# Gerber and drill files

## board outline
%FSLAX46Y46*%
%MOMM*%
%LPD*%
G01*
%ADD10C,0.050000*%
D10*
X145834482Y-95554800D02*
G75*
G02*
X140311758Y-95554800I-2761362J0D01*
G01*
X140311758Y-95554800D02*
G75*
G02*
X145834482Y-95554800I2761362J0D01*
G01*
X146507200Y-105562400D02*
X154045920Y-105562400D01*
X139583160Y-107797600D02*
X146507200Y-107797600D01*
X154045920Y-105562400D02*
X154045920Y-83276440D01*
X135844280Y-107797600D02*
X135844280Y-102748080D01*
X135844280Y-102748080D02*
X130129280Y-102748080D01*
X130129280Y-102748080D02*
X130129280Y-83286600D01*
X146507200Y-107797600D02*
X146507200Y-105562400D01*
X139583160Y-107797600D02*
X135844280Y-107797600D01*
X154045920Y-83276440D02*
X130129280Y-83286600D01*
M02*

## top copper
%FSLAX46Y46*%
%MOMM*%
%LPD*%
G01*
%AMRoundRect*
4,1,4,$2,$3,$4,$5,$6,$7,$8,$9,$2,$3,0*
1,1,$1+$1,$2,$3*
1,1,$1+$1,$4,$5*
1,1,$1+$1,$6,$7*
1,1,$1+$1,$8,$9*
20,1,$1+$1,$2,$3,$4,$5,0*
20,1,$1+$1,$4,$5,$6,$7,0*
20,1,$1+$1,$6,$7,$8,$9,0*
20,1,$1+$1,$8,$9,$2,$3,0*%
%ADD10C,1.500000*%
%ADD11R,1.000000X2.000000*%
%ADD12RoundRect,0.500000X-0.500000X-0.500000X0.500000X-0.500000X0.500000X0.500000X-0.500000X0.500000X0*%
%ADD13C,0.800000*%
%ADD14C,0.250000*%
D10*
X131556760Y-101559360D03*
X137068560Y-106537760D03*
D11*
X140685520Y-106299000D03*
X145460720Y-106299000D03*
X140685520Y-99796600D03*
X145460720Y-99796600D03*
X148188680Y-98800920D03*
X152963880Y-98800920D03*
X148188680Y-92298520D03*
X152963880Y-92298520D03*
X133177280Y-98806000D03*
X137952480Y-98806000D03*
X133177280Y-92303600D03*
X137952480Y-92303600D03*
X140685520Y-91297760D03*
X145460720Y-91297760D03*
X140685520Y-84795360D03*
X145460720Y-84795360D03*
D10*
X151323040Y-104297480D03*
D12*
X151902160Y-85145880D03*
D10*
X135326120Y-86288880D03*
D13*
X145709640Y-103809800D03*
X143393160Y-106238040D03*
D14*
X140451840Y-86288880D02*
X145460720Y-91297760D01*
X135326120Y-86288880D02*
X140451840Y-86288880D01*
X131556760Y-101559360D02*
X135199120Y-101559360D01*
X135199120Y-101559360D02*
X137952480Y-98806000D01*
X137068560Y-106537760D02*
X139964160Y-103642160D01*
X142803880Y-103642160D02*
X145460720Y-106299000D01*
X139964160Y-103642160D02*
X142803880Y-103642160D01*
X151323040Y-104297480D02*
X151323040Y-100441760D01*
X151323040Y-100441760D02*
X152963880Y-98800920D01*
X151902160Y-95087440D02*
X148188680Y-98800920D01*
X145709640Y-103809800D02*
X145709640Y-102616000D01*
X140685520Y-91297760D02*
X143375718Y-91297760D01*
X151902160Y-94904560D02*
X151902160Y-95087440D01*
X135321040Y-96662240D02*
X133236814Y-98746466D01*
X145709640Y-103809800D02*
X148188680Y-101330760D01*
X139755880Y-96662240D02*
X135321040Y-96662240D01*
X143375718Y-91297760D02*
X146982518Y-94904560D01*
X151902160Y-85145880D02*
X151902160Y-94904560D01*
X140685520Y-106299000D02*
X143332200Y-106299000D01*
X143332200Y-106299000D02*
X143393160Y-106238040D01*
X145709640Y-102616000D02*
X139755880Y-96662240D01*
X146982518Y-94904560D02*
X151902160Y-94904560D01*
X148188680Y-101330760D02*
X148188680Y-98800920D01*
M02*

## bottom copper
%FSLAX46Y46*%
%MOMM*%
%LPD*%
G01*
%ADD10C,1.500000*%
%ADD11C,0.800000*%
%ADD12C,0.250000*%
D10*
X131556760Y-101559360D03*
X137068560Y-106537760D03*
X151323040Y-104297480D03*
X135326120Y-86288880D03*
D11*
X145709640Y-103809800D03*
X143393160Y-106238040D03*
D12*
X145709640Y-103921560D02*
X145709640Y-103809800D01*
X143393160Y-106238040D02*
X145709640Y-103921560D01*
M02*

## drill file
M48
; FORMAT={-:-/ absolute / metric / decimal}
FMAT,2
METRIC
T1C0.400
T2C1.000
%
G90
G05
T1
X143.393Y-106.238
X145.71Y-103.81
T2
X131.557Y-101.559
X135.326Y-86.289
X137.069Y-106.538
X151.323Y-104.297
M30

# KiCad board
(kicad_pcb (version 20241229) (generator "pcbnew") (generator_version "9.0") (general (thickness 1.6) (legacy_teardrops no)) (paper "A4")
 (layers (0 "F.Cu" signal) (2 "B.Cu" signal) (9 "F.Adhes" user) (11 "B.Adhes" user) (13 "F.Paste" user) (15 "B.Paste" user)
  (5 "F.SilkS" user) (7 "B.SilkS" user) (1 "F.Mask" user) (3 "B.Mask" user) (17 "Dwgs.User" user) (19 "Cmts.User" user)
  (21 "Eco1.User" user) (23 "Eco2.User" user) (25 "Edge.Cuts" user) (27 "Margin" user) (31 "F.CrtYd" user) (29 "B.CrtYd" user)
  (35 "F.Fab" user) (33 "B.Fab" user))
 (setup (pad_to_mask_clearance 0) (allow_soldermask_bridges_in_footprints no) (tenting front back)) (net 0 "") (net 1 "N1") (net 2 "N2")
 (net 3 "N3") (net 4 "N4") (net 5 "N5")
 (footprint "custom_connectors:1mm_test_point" (layer "F.Cu") (at 131.55676 101.56952)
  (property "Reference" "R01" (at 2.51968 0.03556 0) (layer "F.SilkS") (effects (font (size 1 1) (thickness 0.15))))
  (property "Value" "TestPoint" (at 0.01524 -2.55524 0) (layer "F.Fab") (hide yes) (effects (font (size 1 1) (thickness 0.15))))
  (pad "1" thru_hole circle (at 0 -0.01016) (size 1.5 1.5) (drill 1) (layers "*.Cu" "*.Mask") (remove_unused_layers no) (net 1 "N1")))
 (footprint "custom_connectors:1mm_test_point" (layer "F.Cu") (at 137.06856 106.54792)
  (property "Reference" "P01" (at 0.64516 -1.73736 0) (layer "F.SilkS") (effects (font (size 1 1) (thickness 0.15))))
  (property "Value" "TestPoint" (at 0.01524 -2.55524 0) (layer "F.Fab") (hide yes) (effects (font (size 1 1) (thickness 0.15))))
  (pad "1" thru_hole circle (at 0 -0.01016) (size 1.5 1.5) (drill 1) (layers "*.Cu" "*.Mask") (remove_unused_layers no) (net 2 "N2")))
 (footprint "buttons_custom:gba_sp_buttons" (layer "F.Cu") (at 143.07312 103.0478)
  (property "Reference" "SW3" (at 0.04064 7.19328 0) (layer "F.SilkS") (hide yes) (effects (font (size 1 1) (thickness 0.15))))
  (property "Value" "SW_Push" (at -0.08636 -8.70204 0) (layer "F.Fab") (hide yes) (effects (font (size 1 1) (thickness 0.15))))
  (pad "1" smd rect (at -2.3876 3.2512) (size 1 2) (layers "F.Cu" "F.Mask" "F.Paste") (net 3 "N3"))
  (pad "2" smd rect (at 2.3876 3.2512) (size 1 2) (layers "F.Cu" "F.Mask" "F.Paste") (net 2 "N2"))
  (pad "3" smd rect (at -2.3876 -3.2512) (size 1 2) (layers "F.Cu" "F.Mask" "F.Paste"))
  (pad "4" smd rect (at 2.3876 -3.2512) (size 1 2) (layers "F.Cu" "F.Mask" "F.Paste")))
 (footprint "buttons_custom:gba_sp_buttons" (layer "F.Cu") (at 150.57628 95.54972)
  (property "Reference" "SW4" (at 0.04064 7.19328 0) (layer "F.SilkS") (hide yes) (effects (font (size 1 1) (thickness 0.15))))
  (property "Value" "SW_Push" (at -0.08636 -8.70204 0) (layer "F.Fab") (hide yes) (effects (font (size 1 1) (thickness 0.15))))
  (pad "1" smd rect (at -2.3876 3.2512) (size 1 2) (layers "F.Cu" "F.Mask" "F.Paste") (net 3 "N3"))
  (pad "2" smd rect (at 2.3876 3.2512) (size 1 2) (layers "F.Cu" "F.Mask" "F.Paste") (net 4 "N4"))
  (pad "3" smd rect (at -2.3876 -3.2512) (size 1 2) (layers "F.Cu" "F.Mask" "F.Paste"))
  (pad "4" smd rect (at 2.3876 -3.2512) (size 1 2) (layers "F.Cu" "F.Mask" "F.Paste")))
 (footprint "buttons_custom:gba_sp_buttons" (layer "F.Cu") (at 135.56488 95.5548)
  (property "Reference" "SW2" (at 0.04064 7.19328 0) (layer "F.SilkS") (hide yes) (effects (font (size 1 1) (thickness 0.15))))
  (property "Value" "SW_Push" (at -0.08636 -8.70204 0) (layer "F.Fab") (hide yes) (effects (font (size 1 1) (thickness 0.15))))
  (pad "1" smd rect (at -2.3876 3.2512) (size 1 2) (layers "F.Cu" "F.Mask" "F.Paste") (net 3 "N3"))
  (pad "2" smd rect (at 2.3876 3.2512) (size 1 2) (layers "F.Cu" "F.Mask" "F.Paste") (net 1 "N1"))
  (pad "3" smd rect (at -2.3876 -3.2512) (size 1 2) (layers "F.Cu" "F.Mask" "F.Paste"))
  (pad "4" smd rect (at 2.3876 -3.2512) (size 1 2) (layers "F.Cu" "F.Mask" "F.Paste")))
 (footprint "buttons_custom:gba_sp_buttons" (layer "F.Cu") (at 143.07312 88.04656)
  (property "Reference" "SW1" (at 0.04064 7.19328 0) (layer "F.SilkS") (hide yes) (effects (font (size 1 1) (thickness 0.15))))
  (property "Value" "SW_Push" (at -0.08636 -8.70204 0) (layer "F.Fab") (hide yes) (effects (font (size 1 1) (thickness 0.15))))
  (pad "1" smd rect (at -2.3876 3.2512) (size 1 2) (layers "F.Cu" "F.Mask" "F.Paste") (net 3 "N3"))
  (pad "2" smd rect (at 2.3876 3.2512) (size 1 2) (layers "F.Cu" "F.Mask" "F.Paste") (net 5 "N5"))
  (pad "3" smd rect (at -2.3876 -3.2512) (size 1 2) (layers "F.Cu" "F.Mask" "F.Paste"))
  (pad "4" smd rect (at 2.3876 -3.2512) (size 1 2) (layers "F.Cu" "F.Mask" "F.Paste")))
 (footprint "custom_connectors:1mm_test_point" (layer "F.Cu") (at 151.32304 104.30764)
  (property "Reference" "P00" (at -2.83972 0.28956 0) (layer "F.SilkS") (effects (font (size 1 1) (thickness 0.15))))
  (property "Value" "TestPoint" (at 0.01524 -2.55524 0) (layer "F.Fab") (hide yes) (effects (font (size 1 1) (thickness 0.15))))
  (pad "1" thru_hole circle (at 0 -0.01016) (size 1.5 1.5) (drill 1) (layers "*.Cu" "*.Mask") (remove_unused_layers no) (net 4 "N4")))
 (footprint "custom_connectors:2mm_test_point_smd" (layer "F.Cu") (at 151.90216 85.15604)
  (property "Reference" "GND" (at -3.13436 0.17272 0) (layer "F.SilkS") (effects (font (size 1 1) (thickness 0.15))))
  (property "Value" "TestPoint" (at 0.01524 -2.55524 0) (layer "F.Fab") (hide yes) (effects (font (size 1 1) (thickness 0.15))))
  (pad "1" smd roundrect (at 0 -0.01016) (size 2 2) (layers "F.Cu" "F.Mask" "F.Paste") (roundrect_rratio 0.25) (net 3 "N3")))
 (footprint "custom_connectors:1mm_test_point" (layer "F.Cu") (at 135.32612 86.29904)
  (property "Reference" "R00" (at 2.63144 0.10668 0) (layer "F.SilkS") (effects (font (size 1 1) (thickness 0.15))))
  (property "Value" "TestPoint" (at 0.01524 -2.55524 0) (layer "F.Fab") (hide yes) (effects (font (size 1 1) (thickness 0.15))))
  (pad "1" thru_hole circle (at 0 -0.01016) (size 1.5 1.5) (drill 1) (layers "*.Cu" "*.Mask") (remove_unused_layers no) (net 5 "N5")))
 (gr_circle (center 143.07312 95.5548) (end 145.83156 95.4278) (stroke (width 0.05) (type solid)) (fill no) (layer "Edge.Cuts"))
 (gr_line (start 146.5072 105.5624) (end 154.04592 105.5624) (stroke (width 0.05) (type solid)) (layer "Edge.Cuts"))
 (gr_line (start 139.58316 107.7976) (end 146.5072 107.7976) (stroke (width 0.05) (type solid)) (layer "Edge.Cuts"))
 (gr_line (start 154.04592 105.5624) (end 154.04592 83.27644) (stroke (width 0.05) (type solid)) (layer "Edge.Cuts"))
 (gr_line (start 135.84428 107.7976) (end 135.84428 102.74808) (stroke (width 0.05) (type solid)) (layer "Edge.Cuts"))
 (gr_line (start 135.84428 102.74808) (end 130.12928 102.74808) (stroke (width 0.05) (type solid)) (layer "Edge.Cuts"))
 (gr_line (start 130.12928 102.74808) (end 130.12928 83.2866) (stroke (width 0.05) (type solid)) (layer "Edge.Cuts"))
 (gr_line (start 146.5072 107.7976) (end 146.5072 105.5624) (stroke (width 0.05) (type solid)) (layer "Edge.Cuts"))
 (gr_line (start 139.58316 107.7976) (end 135.84428 107.7976) (stroke (width 0.05) (type solid)) (layer "Edge.Cuts"))
 (gr_line (start 154.04592 83.27644) (end 130.12928 83.2866) (stroke (width 0.05) (type default)) (layer "Edge.Cuts"))
 (segment (start 140.45184 86.28888) (end 145.46072 91.29776) (width 0.25) (layer "F.Cu") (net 5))
 (segment (start 135.32612 86.28888) (end 140.45184 86.28888) (width 0.25) (layer "F.Cu") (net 5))
 (segment (start 131.55676 101.55936) (end 135.19912 101.55936) (width 0.25) (layer "F.Cu") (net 1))
 (segment (start 135.19912 101.55936) (end 137.95248 98.806) (width 0.25) (layer "F.Cu") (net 1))
 (segment (start 137.06856 106.53776) (end 139.96416 103.64216) (width 0.25) (layer "F.Cu") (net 2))
 (segment (start 142.80388 103.64216) (end 145.46072 106.299) (width 0.25) (layer "F.Cu") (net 2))
 (segment (start 139.96416 103.64216) (end 142.80388 103.64216) (width 0.25) (layer "F.Cu") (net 2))
 (segment (start 151.32304 104.29748) (end 151.32304 100.44176) (width 0.25) (layer "F.Cu") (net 4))
 (segment (start 151.32304 100.44176) (end 152.96388 98.80092) (width 0.25) (layer "F.Cu") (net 4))
 (segment (start 151.90216 95.08744) (end 148.18868 98.80092) (width 0.25) (layer "F.Cu") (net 3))
 (segment (start 145.70964 103.8098) (end 145.70964 102.616) (width 0.25) (layer "F.Cu") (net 3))
 (segment (start 140.68552 91.29776) (end 143.375718 91.29776) (width 0.25) (layer "F.Cu") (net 3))
 (segment (start 151.90216 94.90456) (end 151.90216 95.08744) (width 0.25) (layer "F.Cu") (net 3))
 (segment (start 135.32104 96.66224) (end 133.236814 98.746466) (width 0.25) (layer "F.Cu") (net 3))
 (segment (start 145.70964 103.8098) (end 148.18868 101.33076) (width 0.25) (layer "F.Cu") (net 3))
 (segment (start 139.75588 96.66224) (end 135.32104 96.66224) (width 0.25) (layer "F.Cu") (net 3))
 (segment (start 143.375718 91.29776) (end 146.982518 94.90456) (width 0.25) (layer "F.Cu") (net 3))
 (segment (start 151.90216 85.14588) (end 151.90216 94.90456) (width 0.25) (layer "F.Cu") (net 3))
 (segment (start 140.68552 106.299) (end 143.3322 106.299) (width 0.25) (layer "F.Cu") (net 3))
 (segment (start 143.3322 106.299) (end 143.39316 106.23804) (width 0.25) (layer "F.Cu") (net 3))
 (segment (start 145.70964 102.616) (end 139.75588 96.66224) (width 0.25) (layer "F.Cu") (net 3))
 (segment (start 146.982518 94.90456) (end 151.90216 94.90456) (width 0.25) (layer "F.Cu") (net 3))
 (segment (start 148.18868 101.33076) (end 148.18868 98.80092) (width 0.25) (layer "F.Cu") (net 3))
 (via (at 145.70964 103.8098) (size 0.8) (drill 0.4) (layers "F.Cu" "B.Cu") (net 3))
 (via (at 143.39316 106.23804) (size 0.8) (drill 0.4) (layers "F.Cu" "B.Cu") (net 3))
 (segment (start 145.70964 103.92156) (end 145.70964 103.8098) (width 0.25) (layer "B.Cu") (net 3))
 (segment (start 143.39316 106.23804) (end 145.70964 103.92156) (width 0.25) (layer "B.Cu") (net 3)))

